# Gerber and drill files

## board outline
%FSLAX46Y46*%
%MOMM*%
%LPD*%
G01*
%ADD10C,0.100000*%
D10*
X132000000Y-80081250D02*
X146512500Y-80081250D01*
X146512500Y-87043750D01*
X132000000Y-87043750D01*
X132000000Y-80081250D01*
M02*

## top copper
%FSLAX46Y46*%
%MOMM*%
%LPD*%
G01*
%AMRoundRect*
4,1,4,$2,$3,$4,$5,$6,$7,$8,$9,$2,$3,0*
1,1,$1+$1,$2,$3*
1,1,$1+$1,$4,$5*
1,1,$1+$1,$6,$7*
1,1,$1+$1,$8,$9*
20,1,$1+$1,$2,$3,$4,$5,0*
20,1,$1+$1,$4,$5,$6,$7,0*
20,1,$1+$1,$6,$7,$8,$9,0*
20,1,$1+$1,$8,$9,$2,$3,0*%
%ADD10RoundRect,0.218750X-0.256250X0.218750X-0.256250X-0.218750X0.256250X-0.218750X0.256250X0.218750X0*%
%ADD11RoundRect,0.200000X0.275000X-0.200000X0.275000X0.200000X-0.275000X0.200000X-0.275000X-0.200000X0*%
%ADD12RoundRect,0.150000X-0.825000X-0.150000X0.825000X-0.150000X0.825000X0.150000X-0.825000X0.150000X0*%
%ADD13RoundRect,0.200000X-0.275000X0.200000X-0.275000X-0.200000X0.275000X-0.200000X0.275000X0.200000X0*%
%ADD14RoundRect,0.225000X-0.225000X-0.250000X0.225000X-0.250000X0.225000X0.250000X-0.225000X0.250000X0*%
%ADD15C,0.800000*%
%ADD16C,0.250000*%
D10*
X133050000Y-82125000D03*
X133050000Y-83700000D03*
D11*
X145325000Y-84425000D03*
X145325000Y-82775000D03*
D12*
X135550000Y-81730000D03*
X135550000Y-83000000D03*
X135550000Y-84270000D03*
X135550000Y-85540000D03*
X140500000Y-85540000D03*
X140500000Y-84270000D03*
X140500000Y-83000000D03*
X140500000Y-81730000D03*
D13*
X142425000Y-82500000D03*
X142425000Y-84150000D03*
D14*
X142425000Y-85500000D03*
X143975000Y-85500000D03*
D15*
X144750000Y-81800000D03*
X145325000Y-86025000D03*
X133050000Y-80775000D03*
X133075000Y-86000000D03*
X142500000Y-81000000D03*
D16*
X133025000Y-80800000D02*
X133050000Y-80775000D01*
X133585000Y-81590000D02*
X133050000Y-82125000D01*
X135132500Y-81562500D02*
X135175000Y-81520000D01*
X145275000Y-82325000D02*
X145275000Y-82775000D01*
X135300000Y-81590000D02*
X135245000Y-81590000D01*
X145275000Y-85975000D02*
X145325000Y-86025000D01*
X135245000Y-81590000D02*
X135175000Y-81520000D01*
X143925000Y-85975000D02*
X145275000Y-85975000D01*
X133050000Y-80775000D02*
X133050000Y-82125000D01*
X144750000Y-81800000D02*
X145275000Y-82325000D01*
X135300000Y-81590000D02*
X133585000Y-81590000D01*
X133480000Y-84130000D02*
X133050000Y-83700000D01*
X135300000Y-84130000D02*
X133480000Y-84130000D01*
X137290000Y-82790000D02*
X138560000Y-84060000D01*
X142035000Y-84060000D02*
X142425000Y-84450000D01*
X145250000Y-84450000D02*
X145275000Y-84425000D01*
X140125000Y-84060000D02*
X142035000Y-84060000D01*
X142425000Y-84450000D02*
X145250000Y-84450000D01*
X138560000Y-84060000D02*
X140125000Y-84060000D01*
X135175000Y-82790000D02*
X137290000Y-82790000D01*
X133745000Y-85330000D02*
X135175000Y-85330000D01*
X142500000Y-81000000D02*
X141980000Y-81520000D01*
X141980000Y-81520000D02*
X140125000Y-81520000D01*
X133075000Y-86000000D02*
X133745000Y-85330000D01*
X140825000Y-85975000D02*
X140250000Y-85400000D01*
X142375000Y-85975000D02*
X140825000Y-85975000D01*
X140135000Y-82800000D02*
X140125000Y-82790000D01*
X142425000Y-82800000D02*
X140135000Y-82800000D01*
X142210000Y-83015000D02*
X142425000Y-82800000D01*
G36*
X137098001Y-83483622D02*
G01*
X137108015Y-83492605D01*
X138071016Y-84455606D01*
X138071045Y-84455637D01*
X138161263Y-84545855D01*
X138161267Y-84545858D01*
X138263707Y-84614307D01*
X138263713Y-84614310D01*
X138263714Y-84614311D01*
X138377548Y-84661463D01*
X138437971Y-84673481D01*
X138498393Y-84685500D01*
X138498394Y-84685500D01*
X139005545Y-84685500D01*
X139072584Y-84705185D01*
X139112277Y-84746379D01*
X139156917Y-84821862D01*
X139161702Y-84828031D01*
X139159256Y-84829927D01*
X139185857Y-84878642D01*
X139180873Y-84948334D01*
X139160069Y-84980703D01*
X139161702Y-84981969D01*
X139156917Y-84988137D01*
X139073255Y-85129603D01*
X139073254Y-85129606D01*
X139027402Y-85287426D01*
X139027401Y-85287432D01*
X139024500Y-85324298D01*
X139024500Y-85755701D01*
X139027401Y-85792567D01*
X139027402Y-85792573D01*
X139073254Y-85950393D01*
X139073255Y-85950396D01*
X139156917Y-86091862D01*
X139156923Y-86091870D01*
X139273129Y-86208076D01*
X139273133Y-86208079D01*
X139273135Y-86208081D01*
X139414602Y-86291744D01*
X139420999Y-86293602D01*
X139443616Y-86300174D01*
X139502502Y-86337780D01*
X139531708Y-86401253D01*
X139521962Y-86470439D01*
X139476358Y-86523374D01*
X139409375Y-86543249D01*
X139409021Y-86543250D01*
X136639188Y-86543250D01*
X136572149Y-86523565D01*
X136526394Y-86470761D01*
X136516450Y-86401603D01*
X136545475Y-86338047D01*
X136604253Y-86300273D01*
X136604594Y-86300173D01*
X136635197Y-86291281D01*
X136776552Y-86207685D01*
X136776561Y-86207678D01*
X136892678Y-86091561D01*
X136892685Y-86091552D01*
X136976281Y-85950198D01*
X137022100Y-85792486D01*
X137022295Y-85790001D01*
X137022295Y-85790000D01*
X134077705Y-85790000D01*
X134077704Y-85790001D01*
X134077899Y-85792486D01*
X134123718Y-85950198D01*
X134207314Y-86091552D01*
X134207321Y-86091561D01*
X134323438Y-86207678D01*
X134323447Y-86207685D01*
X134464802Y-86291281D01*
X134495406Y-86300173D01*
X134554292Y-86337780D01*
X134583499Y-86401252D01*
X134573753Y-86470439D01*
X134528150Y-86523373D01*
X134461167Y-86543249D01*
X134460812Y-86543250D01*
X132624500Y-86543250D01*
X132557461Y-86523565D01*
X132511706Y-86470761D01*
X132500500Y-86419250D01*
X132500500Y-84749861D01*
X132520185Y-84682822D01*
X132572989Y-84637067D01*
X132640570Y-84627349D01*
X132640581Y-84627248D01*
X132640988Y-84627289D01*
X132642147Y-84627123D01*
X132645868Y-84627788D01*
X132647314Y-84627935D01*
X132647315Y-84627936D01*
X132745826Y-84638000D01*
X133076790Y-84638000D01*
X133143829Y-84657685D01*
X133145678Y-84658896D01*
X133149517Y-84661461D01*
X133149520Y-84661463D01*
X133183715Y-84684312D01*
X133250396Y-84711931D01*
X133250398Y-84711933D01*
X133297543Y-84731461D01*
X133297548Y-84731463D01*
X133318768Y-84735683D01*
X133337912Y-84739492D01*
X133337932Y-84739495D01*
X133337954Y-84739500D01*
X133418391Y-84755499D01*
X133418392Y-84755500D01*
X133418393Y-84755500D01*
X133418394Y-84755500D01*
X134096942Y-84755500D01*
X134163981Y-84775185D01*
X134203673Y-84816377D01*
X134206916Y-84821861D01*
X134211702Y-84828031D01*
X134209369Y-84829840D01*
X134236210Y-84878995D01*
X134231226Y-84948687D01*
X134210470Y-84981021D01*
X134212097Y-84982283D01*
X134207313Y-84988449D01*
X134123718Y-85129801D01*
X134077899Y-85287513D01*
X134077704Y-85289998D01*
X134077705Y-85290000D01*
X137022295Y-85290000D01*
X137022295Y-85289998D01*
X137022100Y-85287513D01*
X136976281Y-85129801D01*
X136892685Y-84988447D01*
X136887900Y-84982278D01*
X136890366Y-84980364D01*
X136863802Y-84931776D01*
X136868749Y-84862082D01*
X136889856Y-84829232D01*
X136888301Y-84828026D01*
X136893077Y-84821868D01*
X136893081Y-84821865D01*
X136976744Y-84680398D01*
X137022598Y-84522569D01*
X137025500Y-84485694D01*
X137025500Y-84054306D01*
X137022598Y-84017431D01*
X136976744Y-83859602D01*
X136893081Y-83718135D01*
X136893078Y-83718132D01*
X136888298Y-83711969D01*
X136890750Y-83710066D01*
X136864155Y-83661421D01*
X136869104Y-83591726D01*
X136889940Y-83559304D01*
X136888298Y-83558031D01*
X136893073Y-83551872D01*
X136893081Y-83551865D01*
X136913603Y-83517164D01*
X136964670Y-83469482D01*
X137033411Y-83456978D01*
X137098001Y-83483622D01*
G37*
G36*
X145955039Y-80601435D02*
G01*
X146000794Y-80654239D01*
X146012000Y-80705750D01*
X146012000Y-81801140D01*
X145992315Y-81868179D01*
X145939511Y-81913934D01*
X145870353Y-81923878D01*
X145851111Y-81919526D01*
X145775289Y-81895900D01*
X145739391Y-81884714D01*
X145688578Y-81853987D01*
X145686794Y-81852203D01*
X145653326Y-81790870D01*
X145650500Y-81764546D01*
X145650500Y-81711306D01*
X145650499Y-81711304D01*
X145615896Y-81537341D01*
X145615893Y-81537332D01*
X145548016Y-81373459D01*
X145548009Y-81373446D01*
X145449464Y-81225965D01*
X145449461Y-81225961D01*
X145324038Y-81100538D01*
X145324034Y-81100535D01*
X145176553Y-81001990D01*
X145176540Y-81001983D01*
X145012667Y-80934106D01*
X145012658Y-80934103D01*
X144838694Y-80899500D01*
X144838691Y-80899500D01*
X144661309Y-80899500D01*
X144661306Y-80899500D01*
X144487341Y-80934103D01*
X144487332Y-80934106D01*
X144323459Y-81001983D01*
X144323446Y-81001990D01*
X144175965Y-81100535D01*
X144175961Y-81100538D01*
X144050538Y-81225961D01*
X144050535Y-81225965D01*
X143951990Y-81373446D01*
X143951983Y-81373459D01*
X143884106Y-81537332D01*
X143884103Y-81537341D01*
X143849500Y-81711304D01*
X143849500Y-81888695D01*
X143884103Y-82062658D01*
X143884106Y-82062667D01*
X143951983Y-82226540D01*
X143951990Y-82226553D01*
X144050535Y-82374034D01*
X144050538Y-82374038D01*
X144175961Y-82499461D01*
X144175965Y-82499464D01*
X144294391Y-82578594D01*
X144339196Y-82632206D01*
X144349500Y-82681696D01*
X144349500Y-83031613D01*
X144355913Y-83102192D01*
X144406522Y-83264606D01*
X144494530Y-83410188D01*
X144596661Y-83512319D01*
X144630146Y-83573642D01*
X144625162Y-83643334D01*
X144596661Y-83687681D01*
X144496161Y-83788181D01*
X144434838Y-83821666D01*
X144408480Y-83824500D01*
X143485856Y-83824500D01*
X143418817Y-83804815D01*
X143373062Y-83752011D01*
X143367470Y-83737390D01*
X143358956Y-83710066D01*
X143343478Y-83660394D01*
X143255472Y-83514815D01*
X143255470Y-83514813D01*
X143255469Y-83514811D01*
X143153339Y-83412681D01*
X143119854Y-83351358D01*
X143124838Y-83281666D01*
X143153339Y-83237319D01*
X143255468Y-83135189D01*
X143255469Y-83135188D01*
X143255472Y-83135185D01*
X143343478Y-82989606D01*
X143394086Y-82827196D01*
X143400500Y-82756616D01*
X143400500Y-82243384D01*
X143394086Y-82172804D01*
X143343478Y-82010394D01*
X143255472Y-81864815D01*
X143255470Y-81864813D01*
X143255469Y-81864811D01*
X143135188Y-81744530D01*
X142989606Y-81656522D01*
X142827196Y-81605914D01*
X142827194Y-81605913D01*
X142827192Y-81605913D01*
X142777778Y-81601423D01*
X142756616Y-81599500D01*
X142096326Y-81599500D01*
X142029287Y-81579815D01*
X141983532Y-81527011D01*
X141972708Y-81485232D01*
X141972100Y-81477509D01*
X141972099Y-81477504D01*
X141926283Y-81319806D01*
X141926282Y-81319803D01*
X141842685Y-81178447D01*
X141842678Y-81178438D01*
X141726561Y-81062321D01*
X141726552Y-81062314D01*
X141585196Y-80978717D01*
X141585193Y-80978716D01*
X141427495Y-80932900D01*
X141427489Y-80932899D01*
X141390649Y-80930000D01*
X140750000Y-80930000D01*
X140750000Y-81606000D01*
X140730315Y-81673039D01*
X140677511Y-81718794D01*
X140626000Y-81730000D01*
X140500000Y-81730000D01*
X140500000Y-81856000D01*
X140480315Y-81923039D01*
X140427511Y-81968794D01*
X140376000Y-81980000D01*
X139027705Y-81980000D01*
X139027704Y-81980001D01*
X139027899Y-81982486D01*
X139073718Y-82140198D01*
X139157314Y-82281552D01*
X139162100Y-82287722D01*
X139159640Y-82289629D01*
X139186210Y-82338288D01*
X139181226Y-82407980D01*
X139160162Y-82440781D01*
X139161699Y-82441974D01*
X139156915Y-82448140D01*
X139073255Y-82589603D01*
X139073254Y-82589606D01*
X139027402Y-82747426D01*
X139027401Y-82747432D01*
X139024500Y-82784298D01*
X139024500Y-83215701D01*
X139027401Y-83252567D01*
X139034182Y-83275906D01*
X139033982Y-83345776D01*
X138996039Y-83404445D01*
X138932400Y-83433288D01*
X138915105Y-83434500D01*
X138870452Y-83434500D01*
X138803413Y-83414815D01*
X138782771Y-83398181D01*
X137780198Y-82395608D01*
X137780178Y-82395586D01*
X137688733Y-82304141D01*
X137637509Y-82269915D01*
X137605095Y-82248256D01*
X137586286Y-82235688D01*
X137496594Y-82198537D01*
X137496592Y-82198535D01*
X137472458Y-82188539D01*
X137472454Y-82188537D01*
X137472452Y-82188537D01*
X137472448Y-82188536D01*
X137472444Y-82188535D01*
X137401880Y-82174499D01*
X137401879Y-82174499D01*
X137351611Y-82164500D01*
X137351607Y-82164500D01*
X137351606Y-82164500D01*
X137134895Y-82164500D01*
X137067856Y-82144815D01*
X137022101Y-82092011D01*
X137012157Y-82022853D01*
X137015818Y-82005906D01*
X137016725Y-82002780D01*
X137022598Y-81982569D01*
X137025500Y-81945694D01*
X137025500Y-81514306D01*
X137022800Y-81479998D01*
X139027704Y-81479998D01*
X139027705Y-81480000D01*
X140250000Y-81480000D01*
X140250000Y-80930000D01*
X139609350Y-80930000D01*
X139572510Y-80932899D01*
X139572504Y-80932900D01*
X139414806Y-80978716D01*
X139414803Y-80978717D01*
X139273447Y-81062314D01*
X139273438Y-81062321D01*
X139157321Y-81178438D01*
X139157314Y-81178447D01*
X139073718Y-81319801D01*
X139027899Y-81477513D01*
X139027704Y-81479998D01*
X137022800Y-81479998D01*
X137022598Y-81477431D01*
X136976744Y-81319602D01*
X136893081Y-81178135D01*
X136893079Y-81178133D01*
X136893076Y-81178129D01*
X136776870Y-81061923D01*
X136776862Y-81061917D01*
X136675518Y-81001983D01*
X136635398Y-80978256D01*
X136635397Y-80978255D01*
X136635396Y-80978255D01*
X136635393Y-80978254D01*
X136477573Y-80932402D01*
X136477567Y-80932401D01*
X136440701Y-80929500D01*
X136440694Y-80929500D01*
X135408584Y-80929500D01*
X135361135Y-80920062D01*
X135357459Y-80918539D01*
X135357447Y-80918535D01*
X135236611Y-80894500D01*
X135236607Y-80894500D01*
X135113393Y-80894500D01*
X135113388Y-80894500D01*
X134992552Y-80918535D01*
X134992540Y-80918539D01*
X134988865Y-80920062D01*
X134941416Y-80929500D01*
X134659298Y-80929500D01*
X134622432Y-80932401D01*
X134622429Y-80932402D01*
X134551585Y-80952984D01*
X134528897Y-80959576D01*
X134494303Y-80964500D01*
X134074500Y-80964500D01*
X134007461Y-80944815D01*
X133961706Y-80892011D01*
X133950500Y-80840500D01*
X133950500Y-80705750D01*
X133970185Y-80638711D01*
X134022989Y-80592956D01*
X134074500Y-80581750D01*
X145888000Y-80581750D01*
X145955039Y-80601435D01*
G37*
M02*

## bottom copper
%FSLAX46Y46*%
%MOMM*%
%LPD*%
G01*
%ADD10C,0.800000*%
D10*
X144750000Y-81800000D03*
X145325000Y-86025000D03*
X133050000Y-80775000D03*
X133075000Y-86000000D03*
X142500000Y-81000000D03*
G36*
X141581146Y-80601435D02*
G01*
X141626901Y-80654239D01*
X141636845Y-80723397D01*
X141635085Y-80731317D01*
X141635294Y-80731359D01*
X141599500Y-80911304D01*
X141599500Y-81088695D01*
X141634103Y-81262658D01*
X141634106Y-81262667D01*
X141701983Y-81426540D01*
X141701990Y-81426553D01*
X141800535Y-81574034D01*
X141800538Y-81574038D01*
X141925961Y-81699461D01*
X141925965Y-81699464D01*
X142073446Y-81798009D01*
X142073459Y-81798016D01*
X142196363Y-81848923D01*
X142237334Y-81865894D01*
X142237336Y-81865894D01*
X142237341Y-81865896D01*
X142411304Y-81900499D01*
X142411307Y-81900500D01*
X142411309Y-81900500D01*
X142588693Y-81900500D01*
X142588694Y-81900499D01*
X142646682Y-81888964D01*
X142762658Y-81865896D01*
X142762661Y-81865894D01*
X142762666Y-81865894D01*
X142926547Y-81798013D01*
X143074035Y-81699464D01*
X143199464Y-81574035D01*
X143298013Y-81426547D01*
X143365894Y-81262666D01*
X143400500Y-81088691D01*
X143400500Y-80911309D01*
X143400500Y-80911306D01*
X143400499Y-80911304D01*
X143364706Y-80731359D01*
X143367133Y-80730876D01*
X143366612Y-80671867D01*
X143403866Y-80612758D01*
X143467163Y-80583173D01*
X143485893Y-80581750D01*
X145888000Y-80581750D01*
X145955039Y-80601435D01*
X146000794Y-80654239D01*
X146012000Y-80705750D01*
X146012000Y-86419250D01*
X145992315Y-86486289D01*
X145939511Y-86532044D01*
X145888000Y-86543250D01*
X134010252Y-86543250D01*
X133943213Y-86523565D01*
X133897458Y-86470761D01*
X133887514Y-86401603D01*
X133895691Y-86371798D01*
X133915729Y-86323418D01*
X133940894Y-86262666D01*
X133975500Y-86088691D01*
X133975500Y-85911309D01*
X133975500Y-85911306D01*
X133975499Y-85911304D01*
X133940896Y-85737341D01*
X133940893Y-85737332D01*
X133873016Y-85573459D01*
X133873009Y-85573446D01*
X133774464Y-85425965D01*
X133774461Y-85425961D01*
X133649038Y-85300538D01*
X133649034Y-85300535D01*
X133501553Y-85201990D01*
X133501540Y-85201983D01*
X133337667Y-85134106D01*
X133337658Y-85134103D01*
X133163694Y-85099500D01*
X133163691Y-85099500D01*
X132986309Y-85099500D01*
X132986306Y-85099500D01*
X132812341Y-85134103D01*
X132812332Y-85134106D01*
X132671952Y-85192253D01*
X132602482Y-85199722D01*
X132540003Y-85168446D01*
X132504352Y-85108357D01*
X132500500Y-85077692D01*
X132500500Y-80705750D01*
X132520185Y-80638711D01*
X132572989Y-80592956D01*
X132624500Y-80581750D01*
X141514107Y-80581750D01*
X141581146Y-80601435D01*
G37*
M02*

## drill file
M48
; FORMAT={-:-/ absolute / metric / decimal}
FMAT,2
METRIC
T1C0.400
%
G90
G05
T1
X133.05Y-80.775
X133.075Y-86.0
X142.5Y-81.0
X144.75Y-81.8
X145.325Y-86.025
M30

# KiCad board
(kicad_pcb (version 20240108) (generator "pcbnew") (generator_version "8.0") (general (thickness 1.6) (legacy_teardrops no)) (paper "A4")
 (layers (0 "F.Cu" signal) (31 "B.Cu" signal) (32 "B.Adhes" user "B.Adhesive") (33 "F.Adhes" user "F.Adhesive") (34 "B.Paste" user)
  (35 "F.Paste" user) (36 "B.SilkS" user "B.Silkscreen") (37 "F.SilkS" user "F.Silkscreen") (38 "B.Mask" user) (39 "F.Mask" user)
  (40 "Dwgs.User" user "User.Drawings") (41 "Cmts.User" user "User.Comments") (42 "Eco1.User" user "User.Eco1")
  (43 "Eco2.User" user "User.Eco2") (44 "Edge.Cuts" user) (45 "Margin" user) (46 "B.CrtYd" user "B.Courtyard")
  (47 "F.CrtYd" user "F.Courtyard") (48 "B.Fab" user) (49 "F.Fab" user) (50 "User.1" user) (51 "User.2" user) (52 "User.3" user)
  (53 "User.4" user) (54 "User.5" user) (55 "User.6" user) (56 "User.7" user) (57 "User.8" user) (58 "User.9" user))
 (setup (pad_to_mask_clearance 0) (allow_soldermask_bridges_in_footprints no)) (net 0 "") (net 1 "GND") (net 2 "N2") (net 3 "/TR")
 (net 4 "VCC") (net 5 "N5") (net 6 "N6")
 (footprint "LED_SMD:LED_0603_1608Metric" (layer "F.Cu") (at 133.05 82.9125 -90)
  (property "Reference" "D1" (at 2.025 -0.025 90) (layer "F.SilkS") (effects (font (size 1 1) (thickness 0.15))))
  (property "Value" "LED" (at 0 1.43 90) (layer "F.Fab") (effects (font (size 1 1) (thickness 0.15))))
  (pad "1" smd roundrect (at -0.7875 0 270) (size 0.875 0.95) (layers "F.Cu" "F.Paste" "F.Mask") (roundrect_rratio 0.25) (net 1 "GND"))
  (pad "2" smd roundrect (at 0.7875 0 270) (size 0.875 0.95) (layers "F.Cu" "F.Paste" "F.Mask") (roundrect_rratio 0.25) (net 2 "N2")))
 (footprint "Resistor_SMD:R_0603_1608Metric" (layer "F.Cu") (at 145.325 83.6 90)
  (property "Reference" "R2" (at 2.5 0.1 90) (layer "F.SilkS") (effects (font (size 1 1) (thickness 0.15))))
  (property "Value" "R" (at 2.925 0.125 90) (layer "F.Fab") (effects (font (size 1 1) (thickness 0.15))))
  (pad "1" smd roundrect (at -0.825 0 90) (size 0.8 0.95) (layers "F.Cu" "F.Paste" "F.Mask") (roundrect_rratio 0.25) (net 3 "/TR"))
  (pad "2" smd roundrect (at 0.825 0 90) (size 0.8 0.95) (layers "F.Cu" "F.Paste" "F.Mask") (roundrect_rratio 0.25) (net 1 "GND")))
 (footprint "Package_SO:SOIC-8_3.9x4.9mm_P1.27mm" (layer "F.Cu") (at 138.025 83.635)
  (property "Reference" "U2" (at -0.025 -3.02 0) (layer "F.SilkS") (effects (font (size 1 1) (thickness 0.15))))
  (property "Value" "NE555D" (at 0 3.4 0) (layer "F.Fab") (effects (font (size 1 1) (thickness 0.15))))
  (pad "1" smd roundrect (at -2.475 -1.905) (size 1.95 0.6) (layers "F.Cu" "F.Paste" "F.Mask") (roundrect_rratio 0.25) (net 1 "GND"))
  (pad "2" smd roundrect (at -2.475 -0.635) (size 1.95 0.6) (layers "F.Cu" "F.Paste" "F.Mask") (roundrect_rratio 0.25) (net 3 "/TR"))
  (pad "3" smd roundrect (at -2.475 0.635) (size 1.95 0.6) (layers "F.Cu" "F.Paste" "F.Mask") (roundrect_rratio 0.25) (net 2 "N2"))
  (pad "4" smd roundrect (at -2.475 1.905) (size 1.95 0.6) (layers "F.Cu" "F.Paste" "F.Mask") (roundrect_rratio 0.25) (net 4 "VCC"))
  (pad "5" smd roundrect (at 2.475 1.905) (size 1.95 0.6) (layers "F.Cu" "F.Paste" "F.Mask") (roundrect_rratio 0.25) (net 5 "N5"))
  (pad "6" smd roundrect (at 2.475 0.635) (size 1.95 0.6) (layers "F.Cu" "F.Paste" "F.Mask") (roundrect_rratio 0.25) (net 3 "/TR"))
  (pad "7" smd roundrect (at 2.475 -0.635) (size 1.95 0.6) (layers "F.Cu" "F.Paste" "F.Mask") (roundrect_rratio 0.25) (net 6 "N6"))
  (pad "8" smd roundrect (at 2.475 -1.905) (size 1.95 0.6) (layers "F.Cu" "F.Paste" "F.Mask") (roundrect_rratio 0.25) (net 4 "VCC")))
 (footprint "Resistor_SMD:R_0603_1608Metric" (layer "F.Cu") (at 142.425 83.325 -90)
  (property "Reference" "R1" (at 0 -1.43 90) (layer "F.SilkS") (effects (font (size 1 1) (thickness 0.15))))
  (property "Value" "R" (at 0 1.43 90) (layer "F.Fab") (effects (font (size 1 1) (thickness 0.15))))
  (pad "1" smd roundrect (at -0.825 0 270) (size 0.8 0.95) (layers "F.Cu" "F.Paste" "F.Mask") (roundrect_rratio 0.25) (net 6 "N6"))
  (pad "2" smd roundrect (at 0.825 0 270) (size 0.8 0.95) (layers "F.Cu" "F.Paste" "F.Mask") (roundrect_rratio 0.25) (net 3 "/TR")))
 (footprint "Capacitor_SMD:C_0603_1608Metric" (layer "F.Cu") (at 143.2 85.5)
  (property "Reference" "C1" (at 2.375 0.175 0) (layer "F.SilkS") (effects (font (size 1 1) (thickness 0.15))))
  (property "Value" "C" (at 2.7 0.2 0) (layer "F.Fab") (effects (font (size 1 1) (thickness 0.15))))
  (pad "1" smd roundrect (at -0.775 0) (size 0.9 0.95) (layers "F.Cu" "F.Paste" "F.Mask") (roundrect_rratio 0.25) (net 5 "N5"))
  (pad "2" smd roundrect (at 0.775 0) (size 0.9 0.95) (layers "F.Cu" "F.Paste" "F.Mask") (roundrect_rratio 0.25) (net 1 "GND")))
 (gr_rect (start 132 80.08125) (end 146.5125 87.04375) (stroke (width 0.1) (type default)) (fill none) (layer "Edge.Cuts"))
 (segment (start 133.025 80.8) (end 133.05 80.775) (width 0.25) (layer "F.Cu") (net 1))
 (segment (start 133.585 81.59) (end 133.05 82.125) (width 0.25) (layer "F.Cu") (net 1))
 (segment (start 135.1325 81.5625) (end 135.175 81.52) (width 0.25) (layer "F.Cu") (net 1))
 (segment (start 145.275 82.325) (end 145.275 82.775) (width 0.25) (layer "F.Cu") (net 1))
 (segment (start 135.3 81.59) (end 135.245 81.59) (width 0.25) (layer "F.Cu") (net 1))
 (segment (start 145.275 85.975) (end 145.325 86.025) (width 0.25) (layer "F.Cu") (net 1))
 (segment (start 135.245 81.59) (end 135.175 81.52) (width 0.25) (layer "F.Cu") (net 1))
 (segment (start 143.925 85.975) (end 145.275 85.975) (width 0.25) (layer "F.Cu") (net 1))
 (segment (start 133.05 80.775) (end 133.05 82.125) (width 0.25) (layer "F.Cu") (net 1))
 (segment (start 144.75 81.8) (end 145.275 82.325) (width 0.25) (layer "F.Cu") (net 1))
 (segment (start 135.3 81.59) (end 133.585 81.59) (width 0.25) (layer "F.Cu") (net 1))
 (via (at 144.75 81.8) (size 0.8) (drill 0.4) (layers "F.Cu" "B.Cu") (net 1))
 (via (at 145.325 86.025) (size 0.8) (drill 0.4) (layers "F.Cu" "B.Cu") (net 1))
 (via (at 133.05 80.775) (size 0.8) (drill 0.4) (layers "F.Cu" "B.Cu") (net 1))
 (segment (start 133.48 84.13) (end 133.05 83.7) (width 0.25) (layer "F.Cu") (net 2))
 (segment (start 135.3 84.13) (end 133.48 84.13) (width 0.25) (layer "F.Cu") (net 2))
 (segment (start 137.29 82.79) (end 138.56 84.06) (width 0.25) (layer "F.Cu") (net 3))
 (segment (start 142.035 84.06) (end 142.425 84.45) (width 0.25) (layer "F.Cu") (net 3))
 (segment (start 145.25 84.45) (end 145.275 84.425) (width 0.25) (layer "F.Cu") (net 3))
 (segment (start 140.125 84.06) (end 142.035 84.06) (width 0.25) (layer "F.Cu") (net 3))
 (segment (start 142.425 84.45) (end 145.25 84.45) (width 0.25) (layer "F.Cu") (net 3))
 (segment (start 138.56 84.06) (end 140.125 84.06) (width 0.25) (layer "F.Cu") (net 3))
 (segment (start 135.175 82.79) (end 137.29 82.79) (width 0.25) (layer "F.Cu") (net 3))
 (segment (start 133.745 85.33) (end 135.175 85.33) (width 0.25) (layer "F.Cu") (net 4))
 (segment (start 142.5 81) (end 141.98 81.52) (width 0.25) (layer "F.Cu") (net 4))
 (segment (start 141.98 81.52) (end 140.125 81.52) (width 0.25) (layer "F.Cu") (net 4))
 (segment (start 133.075 86) (end 133.745 85.33) (width 0.25) (layer "F.Cu") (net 4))
 (via (at 133.075 86) (size 0.8) (drill 0.4) (layers "F.Cu" "B.Cu") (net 4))
 (via (at 142.5 81) (size 0.8) (drill 0.4) (layers "F.Cu" "B.Cu") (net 4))
 (segment (start 140.825 85.975) (end 140.25 85.4) (width 0.25) (layer "F.Cu") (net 5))
 (segment (start 142.375 85.975) (end 140.825 85.975) (width 0.25) (layer "F.Cu") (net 5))
 (segment (start 140.135 82.8) (end 140.125 82.79) (width 0.25) (layer "F.Cu") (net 6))
 (segment (start 142.425 82.8) (end 140.135 82.8) (width 0.25) (layer "F.Cu") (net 6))
 (segment (start 142.21 83.015) (end 142.425 82.8) (width 0.25) (layer "F.Cu") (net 6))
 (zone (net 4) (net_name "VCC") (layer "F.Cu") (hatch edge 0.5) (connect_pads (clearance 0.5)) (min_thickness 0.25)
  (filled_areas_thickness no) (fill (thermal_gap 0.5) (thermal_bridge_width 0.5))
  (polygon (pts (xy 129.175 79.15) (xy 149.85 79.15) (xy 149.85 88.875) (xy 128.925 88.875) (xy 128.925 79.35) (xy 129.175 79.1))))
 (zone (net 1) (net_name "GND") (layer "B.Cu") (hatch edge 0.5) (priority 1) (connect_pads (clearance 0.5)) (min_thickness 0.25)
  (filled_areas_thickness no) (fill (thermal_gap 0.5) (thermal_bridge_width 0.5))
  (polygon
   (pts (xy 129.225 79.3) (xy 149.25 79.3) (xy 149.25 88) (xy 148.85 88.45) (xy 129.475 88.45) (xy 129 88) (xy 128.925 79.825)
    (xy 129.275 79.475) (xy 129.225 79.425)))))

